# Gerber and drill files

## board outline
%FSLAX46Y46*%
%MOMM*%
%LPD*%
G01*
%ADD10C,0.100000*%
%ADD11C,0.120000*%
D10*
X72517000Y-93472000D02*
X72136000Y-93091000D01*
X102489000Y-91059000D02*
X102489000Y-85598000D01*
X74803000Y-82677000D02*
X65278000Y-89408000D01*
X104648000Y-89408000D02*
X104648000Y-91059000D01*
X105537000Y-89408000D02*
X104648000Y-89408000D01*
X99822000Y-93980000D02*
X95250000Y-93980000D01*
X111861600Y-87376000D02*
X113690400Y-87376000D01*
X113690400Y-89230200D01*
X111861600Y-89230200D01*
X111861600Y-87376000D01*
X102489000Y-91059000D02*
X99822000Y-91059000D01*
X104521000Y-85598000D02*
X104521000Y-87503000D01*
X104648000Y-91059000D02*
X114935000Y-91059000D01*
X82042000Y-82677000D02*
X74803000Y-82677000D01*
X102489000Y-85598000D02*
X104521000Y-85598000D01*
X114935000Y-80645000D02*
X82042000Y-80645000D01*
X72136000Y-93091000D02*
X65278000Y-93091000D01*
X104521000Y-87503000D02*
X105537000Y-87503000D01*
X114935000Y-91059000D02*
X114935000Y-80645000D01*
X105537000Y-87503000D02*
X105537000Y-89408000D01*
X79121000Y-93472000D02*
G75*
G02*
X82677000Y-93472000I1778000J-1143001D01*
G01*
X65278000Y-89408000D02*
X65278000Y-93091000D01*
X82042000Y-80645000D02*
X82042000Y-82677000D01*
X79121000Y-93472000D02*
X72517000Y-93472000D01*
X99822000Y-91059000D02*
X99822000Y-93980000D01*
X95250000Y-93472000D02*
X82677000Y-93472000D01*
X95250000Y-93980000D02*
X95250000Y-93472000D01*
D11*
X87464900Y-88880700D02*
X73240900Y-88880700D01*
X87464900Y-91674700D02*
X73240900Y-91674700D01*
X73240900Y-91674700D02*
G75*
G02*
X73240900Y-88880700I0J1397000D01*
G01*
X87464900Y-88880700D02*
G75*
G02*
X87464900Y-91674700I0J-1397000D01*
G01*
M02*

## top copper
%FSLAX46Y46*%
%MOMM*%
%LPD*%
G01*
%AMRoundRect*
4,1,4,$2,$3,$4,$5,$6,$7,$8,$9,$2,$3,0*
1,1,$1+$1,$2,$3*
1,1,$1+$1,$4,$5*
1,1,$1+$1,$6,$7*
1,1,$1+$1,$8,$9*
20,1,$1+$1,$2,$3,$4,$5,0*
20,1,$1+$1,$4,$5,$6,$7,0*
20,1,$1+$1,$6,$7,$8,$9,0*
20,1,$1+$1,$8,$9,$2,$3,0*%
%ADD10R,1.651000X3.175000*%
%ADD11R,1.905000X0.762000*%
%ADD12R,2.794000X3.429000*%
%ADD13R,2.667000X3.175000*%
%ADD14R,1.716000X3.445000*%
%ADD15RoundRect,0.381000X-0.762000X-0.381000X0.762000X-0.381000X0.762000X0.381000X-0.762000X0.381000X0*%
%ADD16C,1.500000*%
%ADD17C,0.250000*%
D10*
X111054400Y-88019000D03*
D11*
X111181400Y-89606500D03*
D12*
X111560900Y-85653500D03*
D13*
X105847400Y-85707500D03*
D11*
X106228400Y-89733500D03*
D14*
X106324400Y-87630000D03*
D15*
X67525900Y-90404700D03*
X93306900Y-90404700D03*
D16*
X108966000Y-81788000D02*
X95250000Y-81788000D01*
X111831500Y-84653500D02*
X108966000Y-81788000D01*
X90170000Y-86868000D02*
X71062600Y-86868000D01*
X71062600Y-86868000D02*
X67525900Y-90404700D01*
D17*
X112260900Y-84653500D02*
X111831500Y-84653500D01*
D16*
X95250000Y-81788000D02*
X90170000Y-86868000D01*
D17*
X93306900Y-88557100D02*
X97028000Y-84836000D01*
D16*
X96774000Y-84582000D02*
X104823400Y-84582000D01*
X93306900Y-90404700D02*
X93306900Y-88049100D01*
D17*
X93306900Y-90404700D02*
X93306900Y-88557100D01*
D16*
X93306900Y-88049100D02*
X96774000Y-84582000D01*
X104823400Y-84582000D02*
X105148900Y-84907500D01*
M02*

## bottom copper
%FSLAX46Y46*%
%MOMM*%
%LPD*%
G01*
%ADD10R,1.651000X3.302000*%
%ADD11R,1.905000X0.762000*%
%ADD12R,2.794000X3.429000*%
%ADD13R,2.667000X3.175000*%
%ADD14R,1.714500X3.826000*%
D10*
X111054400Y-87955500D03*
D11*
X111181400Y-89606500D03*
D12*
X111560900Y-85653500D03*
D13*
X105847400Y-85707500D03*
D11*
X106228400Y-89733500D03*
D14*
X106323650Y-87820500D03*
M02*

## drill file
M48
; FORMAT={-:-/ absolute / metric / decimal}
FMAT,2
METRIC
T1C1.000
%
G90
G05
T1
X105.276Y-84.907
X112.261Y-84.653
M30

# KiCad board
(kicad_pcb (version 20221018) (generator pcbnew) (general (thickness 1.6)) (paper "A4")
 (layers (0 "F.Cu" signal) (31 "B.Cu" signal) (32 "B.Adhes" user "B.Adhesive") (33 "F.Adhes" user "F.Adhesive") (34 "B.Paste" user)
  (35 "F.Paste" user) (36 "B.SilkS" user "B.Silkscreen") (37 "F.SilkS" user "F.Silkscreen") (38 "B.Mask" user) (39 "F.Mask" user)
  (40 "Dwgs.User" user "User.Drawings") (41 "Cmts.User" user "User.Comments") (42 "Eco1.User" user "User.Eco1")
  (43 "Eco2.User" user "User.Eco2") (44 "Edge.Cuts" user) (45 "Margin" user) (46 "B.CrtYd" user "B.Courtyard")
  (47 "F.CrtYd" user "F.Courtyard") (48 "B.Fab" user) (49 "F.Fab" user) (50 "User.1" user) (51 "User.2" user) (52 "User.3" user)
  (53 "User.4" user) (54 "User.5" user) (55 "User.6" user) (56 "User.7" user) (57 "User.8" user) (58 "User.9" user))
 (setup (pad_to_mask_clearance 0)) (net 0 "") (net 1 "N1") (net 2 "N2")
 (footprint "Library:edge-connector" (layer "F.Cu") (at 108.4509 77.7955)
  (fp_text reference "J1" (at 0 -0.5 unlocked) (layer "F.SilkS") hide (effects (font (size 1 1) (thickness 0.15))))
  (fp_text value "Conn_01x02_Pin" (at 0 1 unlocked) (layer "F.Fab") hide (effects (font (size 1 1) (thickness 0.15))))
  (pad "1" smd rect (at 2.6035 10.16) (size 1.651 3.302) (layers "B.Cu" "B.Paste" "B.Mask") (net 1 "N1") (thermal_bridge_angle 45))
  (pad "1" smd rect (at 2.6035 10.2235) (size 1.651 3.175) (layers "F.Cu" "F.Paste" "F.Mask") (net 1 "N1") (thermal_bridge_angle 45))
  (pad "1" smd rect (at 2.7305 11.811) (size 1.905 0.762) (layers "F.Cu" "F.Paste" "F.Mask") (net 1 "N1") (thermal_bridge_angle 45))
  (pad "1" smd rect (at 2.7305 11.811) (size 1.905 0.762) (layers "B.Cu" "B.Paste" "B.Mask") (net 1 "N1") (thermal_bridge_angle 45))
  (pad "1" thru_hole rect (at 3.81 6.858) (size 2.794 3.429) (drill 1 (offset -0.7 1)) (layers "*.Cu" "*.Mask") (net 1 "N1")
   (thermal_bridge_angle 45))
  (pad "2" thru_hole rect (at -3.175 7.112) (size 2.667 3.175) (drill 1 (offset 0.5715 0.8)) (layers "*.Cu" "*.Mask") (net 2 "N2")
   (thermal_bridge_angle 45))
  (pad "2" smd rect (at -2.2225 11.938) (size 1.905 0.762) (layers "F.Cu" "F.Paste" "F.Mask") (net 2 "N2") (thermal_bridge_angle 45))
  (pad "2" smd rect (at -2.2225 11.938) (size 1.905 0.762) (layers "B.Cu" "B.Paste" "B.Mask") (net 2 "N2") (thermal_bridge_angle 45))
  (pad "2" smd rect (at -2.12725 10.025) (size 1.7145 3.826) (layers "B.Cu" "B.Paste" "B.Mask") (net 2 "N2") (thermal_bridge_angle 45))
  (pad "2" smd rect (at -2.1265 9.8345) (size 1.716 3.445) (layers "F.Cu" "F.Paste" "F.Mask") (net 2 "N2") (thermal_bridge_angle 45)))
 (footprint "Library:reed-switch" (layer "F.Cu") (at 81.1149 84.4357)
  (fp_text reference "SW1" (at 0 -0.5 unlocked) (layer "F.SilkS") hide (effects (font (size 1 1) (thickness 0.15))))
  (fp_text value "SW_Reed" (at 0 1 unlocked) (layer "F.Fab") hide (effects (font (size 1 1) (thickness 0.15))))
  (fp_line (start 6.35 4.445) (end -7.874 4.445) (stroke (width 0.12) (type default)) (layer "Edge.Cuts"))
  (fp_line (start 6.35 7.239) (end -7.874 7.239) (stroke (width 0.12) (type default)) (layer "Edge.Cuts"))
  (fp_arc (start -7.874 7.239) (mid -9.271 5.842) (end -7.874 4.445) (stroke (width 0.12) (type default)) (layer "Edge.Cuts"))
  (fp_arc (start 6.35 4.445) (mid 7.747 5.842) (end 6.35 7.239) (stroke (width 0.12) (type default)) (layer "Edge.Cuts"))
  (pad "1" smd roundrect (at -13.589 5.969) (size 2.286 1.524) (layers "F.Cu" "F.Paste" "F.Mask") (roundrect_rratio 0.25) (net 1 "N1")
   (thermal_bridge_angle 45))
  (pad "2" smd roundrect (at 12.192 5.969) (size 2.286 1.524) (layers "F.Cu" "F.Paste" "F.Mask") (roundrect_rratio 0.25) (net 2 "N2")
   (thermal_bridge_angle 45)))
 (gr_line (start 72.517 93.472) (end 72.136 93.091) (stroke (width 0.1) (type default)) (layer "Edge.Cuts"))
 (gr_line (start 102.489 91.059) (end 102.489 85.598) (stroke (width 0.1) (type default)) (layer "Edge.Cuts"))
 (gr_line (start 74.803 82.677) (end 65.278 89.408) (stroke (width 0.1) (type default)) (layer "Edge.Cuts"))
 (gr_line (start 104.648 89.408) (end 104.648 91.059) (stroke (width 0.1) (type default)) (layer "Edge.Cuts"))
 (gr_line (start 105.537 89.408) (end 104.648 89.408) (stroke (width 0.1) (type default)) (layer "Edge.Cuts"))
 (gr_line (start 99.822 93.98) (end 95.25 93.98) (stroke (width 0.1) (type default)) (layer "Edge.Cuts"))
 (gr_rect (start 111.8616 87.376) (end 113.6904 89.2302) (stroke (width 0.1) (type default)) (fill none) (layer "Edge.Cuts"))
 (gr_line (start 102.489 91.059) (end 99.822 91.059) (stroke (width 0.1) (type default)) (layer "Edge.Cuts"))
 (gr_line (start 104.521 85.598) (end 104.521 87.503) (stroke (width 0.1) (type default)) (layer "Edge.Cuts"))
 (gr_line (start 104.648 91.059) (end 114.935 91.059) (stroke (width 0.1) (type default)) (layer "Edge.Cuts"))
 (gr_line (start 82.042 82.677) (end 74.803 82.677) (stroke (width 0.1) (type default)) (layer "Edge.Cuts"))
 (gr_line (start 102.489 85.598) (end 104.521 85.598) (stroke (width 0.1) (type default)) (layer "Edge.Cuts"))
 (gr_line (start 114.935 80.645) (end 82.042 80.645) (stroke (width 0.1) (type default)) (layer "Edge.Cuts"))
 (gr_line (start 72.136 93.091) (end 65.278 93.091) (stroke (width 0.1) (type default)) (layer "Edge.Cuts"))
 (gr_line (start 104.521 87.503) (end 105.537 87.503) (stroke (width 0.1) (type default)) (layer "Edge.Cuts"))
 (gr_line (start 114.935 91.059) (end 114.935 80.645) (stroke (width 0.1) (type default)) (layer "Edge.Cuts"))
 (gr_line (start 105.537 87.503) (end 105.537 89.408) (stroke (width 0.1) (type default)) (layer "Edge.Cuts"))
 (gr_arc (start 79.121 93.472) (mid 80.899 92.501299) (end 82.677 93.472) (stroke (width 0.1) (type default)) (layer "Edge.Cuts"))
 (gr_line (start 65.278 89.408) (end 65.278 93.091) (stroke (width 0.1) (type default)) (layer "Edge.Cuts"))
 (gr_line (start 82.042 80.645) (end 82.042 82.677) (stroke (width 0.1) (type default)) (layer "Edge.Cuts"))
 (gr_line (start 79.121 93.472) (end 72.517 93.472) (stroke (width 0.1) (type default)) (layer "Edge.Cuts"))
 (gr_line (start 99.822 91.059) (end 99.822 93.98) (stroke (width 0.1) (type default)) (layer "Edge.Cuts"))
 (gr_line (start 95.25 93.472) (end 82.677 93.472) (stroke (width 0.1) (type default)) (layer "Edge.Cuts"))
 (gr_line (start 95.25 93.98) (end 95.25 93.472) (stroke (width 0.1) (type default)) (layer "Edge.Cuts"))
 (segment (start 108.966 81.788) (end 95.25 81.788) (width 1.5) (layer "F.Cu") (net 1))
 (segment (start 111.8315 84.6535) (end 108.966 81.788) (width 1.5) (layer "F.Cu") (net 1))
 (segment (start 90.17 86.868) (end 71.0626 86.868) (width 1.5) (layer "F.Cu") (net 1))
 (segment (start 71.0626 86.868) (end 67.5259 90.4047) (width 1.5) (layer "F.Cu") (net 1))
 (segment (start 112.2609 84.6535) (end 111.8315 84.6535) (width 0.25) (layer "F.Cu") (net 1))
 (segment (start 95.25 81.788) (end 90.17 86.868) (width 1.5) (layer "F.Cu") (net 1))
 (segment (start 93.3069 88.5571) (end 97.028 84.836) (width 0.25) (layer "F.Cu") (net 2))
 (segment (start 96.774 84.582) (end 104.8234 84.582) (width 1.5) (layer "F.Cu") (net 2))
 (segment (start 93.3069 90.4047) (end 93.3069 88.0491) (width 1.5) (layer "F.Cu") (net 2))
 (segment (start 93.3069 90.4047) (end 93.3069 88.5571) (width 0.25) (layer "F.Cu") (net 2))
 (segment (start 93.3069 88.0491) (end 96.774 84.582) (width 1.5) (layer "F.Cu") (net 2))
 (segment (start 104.8234 84.582) (end 105.1489 84.9075) (width 1.5) (layer "F.Cu") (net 2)))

